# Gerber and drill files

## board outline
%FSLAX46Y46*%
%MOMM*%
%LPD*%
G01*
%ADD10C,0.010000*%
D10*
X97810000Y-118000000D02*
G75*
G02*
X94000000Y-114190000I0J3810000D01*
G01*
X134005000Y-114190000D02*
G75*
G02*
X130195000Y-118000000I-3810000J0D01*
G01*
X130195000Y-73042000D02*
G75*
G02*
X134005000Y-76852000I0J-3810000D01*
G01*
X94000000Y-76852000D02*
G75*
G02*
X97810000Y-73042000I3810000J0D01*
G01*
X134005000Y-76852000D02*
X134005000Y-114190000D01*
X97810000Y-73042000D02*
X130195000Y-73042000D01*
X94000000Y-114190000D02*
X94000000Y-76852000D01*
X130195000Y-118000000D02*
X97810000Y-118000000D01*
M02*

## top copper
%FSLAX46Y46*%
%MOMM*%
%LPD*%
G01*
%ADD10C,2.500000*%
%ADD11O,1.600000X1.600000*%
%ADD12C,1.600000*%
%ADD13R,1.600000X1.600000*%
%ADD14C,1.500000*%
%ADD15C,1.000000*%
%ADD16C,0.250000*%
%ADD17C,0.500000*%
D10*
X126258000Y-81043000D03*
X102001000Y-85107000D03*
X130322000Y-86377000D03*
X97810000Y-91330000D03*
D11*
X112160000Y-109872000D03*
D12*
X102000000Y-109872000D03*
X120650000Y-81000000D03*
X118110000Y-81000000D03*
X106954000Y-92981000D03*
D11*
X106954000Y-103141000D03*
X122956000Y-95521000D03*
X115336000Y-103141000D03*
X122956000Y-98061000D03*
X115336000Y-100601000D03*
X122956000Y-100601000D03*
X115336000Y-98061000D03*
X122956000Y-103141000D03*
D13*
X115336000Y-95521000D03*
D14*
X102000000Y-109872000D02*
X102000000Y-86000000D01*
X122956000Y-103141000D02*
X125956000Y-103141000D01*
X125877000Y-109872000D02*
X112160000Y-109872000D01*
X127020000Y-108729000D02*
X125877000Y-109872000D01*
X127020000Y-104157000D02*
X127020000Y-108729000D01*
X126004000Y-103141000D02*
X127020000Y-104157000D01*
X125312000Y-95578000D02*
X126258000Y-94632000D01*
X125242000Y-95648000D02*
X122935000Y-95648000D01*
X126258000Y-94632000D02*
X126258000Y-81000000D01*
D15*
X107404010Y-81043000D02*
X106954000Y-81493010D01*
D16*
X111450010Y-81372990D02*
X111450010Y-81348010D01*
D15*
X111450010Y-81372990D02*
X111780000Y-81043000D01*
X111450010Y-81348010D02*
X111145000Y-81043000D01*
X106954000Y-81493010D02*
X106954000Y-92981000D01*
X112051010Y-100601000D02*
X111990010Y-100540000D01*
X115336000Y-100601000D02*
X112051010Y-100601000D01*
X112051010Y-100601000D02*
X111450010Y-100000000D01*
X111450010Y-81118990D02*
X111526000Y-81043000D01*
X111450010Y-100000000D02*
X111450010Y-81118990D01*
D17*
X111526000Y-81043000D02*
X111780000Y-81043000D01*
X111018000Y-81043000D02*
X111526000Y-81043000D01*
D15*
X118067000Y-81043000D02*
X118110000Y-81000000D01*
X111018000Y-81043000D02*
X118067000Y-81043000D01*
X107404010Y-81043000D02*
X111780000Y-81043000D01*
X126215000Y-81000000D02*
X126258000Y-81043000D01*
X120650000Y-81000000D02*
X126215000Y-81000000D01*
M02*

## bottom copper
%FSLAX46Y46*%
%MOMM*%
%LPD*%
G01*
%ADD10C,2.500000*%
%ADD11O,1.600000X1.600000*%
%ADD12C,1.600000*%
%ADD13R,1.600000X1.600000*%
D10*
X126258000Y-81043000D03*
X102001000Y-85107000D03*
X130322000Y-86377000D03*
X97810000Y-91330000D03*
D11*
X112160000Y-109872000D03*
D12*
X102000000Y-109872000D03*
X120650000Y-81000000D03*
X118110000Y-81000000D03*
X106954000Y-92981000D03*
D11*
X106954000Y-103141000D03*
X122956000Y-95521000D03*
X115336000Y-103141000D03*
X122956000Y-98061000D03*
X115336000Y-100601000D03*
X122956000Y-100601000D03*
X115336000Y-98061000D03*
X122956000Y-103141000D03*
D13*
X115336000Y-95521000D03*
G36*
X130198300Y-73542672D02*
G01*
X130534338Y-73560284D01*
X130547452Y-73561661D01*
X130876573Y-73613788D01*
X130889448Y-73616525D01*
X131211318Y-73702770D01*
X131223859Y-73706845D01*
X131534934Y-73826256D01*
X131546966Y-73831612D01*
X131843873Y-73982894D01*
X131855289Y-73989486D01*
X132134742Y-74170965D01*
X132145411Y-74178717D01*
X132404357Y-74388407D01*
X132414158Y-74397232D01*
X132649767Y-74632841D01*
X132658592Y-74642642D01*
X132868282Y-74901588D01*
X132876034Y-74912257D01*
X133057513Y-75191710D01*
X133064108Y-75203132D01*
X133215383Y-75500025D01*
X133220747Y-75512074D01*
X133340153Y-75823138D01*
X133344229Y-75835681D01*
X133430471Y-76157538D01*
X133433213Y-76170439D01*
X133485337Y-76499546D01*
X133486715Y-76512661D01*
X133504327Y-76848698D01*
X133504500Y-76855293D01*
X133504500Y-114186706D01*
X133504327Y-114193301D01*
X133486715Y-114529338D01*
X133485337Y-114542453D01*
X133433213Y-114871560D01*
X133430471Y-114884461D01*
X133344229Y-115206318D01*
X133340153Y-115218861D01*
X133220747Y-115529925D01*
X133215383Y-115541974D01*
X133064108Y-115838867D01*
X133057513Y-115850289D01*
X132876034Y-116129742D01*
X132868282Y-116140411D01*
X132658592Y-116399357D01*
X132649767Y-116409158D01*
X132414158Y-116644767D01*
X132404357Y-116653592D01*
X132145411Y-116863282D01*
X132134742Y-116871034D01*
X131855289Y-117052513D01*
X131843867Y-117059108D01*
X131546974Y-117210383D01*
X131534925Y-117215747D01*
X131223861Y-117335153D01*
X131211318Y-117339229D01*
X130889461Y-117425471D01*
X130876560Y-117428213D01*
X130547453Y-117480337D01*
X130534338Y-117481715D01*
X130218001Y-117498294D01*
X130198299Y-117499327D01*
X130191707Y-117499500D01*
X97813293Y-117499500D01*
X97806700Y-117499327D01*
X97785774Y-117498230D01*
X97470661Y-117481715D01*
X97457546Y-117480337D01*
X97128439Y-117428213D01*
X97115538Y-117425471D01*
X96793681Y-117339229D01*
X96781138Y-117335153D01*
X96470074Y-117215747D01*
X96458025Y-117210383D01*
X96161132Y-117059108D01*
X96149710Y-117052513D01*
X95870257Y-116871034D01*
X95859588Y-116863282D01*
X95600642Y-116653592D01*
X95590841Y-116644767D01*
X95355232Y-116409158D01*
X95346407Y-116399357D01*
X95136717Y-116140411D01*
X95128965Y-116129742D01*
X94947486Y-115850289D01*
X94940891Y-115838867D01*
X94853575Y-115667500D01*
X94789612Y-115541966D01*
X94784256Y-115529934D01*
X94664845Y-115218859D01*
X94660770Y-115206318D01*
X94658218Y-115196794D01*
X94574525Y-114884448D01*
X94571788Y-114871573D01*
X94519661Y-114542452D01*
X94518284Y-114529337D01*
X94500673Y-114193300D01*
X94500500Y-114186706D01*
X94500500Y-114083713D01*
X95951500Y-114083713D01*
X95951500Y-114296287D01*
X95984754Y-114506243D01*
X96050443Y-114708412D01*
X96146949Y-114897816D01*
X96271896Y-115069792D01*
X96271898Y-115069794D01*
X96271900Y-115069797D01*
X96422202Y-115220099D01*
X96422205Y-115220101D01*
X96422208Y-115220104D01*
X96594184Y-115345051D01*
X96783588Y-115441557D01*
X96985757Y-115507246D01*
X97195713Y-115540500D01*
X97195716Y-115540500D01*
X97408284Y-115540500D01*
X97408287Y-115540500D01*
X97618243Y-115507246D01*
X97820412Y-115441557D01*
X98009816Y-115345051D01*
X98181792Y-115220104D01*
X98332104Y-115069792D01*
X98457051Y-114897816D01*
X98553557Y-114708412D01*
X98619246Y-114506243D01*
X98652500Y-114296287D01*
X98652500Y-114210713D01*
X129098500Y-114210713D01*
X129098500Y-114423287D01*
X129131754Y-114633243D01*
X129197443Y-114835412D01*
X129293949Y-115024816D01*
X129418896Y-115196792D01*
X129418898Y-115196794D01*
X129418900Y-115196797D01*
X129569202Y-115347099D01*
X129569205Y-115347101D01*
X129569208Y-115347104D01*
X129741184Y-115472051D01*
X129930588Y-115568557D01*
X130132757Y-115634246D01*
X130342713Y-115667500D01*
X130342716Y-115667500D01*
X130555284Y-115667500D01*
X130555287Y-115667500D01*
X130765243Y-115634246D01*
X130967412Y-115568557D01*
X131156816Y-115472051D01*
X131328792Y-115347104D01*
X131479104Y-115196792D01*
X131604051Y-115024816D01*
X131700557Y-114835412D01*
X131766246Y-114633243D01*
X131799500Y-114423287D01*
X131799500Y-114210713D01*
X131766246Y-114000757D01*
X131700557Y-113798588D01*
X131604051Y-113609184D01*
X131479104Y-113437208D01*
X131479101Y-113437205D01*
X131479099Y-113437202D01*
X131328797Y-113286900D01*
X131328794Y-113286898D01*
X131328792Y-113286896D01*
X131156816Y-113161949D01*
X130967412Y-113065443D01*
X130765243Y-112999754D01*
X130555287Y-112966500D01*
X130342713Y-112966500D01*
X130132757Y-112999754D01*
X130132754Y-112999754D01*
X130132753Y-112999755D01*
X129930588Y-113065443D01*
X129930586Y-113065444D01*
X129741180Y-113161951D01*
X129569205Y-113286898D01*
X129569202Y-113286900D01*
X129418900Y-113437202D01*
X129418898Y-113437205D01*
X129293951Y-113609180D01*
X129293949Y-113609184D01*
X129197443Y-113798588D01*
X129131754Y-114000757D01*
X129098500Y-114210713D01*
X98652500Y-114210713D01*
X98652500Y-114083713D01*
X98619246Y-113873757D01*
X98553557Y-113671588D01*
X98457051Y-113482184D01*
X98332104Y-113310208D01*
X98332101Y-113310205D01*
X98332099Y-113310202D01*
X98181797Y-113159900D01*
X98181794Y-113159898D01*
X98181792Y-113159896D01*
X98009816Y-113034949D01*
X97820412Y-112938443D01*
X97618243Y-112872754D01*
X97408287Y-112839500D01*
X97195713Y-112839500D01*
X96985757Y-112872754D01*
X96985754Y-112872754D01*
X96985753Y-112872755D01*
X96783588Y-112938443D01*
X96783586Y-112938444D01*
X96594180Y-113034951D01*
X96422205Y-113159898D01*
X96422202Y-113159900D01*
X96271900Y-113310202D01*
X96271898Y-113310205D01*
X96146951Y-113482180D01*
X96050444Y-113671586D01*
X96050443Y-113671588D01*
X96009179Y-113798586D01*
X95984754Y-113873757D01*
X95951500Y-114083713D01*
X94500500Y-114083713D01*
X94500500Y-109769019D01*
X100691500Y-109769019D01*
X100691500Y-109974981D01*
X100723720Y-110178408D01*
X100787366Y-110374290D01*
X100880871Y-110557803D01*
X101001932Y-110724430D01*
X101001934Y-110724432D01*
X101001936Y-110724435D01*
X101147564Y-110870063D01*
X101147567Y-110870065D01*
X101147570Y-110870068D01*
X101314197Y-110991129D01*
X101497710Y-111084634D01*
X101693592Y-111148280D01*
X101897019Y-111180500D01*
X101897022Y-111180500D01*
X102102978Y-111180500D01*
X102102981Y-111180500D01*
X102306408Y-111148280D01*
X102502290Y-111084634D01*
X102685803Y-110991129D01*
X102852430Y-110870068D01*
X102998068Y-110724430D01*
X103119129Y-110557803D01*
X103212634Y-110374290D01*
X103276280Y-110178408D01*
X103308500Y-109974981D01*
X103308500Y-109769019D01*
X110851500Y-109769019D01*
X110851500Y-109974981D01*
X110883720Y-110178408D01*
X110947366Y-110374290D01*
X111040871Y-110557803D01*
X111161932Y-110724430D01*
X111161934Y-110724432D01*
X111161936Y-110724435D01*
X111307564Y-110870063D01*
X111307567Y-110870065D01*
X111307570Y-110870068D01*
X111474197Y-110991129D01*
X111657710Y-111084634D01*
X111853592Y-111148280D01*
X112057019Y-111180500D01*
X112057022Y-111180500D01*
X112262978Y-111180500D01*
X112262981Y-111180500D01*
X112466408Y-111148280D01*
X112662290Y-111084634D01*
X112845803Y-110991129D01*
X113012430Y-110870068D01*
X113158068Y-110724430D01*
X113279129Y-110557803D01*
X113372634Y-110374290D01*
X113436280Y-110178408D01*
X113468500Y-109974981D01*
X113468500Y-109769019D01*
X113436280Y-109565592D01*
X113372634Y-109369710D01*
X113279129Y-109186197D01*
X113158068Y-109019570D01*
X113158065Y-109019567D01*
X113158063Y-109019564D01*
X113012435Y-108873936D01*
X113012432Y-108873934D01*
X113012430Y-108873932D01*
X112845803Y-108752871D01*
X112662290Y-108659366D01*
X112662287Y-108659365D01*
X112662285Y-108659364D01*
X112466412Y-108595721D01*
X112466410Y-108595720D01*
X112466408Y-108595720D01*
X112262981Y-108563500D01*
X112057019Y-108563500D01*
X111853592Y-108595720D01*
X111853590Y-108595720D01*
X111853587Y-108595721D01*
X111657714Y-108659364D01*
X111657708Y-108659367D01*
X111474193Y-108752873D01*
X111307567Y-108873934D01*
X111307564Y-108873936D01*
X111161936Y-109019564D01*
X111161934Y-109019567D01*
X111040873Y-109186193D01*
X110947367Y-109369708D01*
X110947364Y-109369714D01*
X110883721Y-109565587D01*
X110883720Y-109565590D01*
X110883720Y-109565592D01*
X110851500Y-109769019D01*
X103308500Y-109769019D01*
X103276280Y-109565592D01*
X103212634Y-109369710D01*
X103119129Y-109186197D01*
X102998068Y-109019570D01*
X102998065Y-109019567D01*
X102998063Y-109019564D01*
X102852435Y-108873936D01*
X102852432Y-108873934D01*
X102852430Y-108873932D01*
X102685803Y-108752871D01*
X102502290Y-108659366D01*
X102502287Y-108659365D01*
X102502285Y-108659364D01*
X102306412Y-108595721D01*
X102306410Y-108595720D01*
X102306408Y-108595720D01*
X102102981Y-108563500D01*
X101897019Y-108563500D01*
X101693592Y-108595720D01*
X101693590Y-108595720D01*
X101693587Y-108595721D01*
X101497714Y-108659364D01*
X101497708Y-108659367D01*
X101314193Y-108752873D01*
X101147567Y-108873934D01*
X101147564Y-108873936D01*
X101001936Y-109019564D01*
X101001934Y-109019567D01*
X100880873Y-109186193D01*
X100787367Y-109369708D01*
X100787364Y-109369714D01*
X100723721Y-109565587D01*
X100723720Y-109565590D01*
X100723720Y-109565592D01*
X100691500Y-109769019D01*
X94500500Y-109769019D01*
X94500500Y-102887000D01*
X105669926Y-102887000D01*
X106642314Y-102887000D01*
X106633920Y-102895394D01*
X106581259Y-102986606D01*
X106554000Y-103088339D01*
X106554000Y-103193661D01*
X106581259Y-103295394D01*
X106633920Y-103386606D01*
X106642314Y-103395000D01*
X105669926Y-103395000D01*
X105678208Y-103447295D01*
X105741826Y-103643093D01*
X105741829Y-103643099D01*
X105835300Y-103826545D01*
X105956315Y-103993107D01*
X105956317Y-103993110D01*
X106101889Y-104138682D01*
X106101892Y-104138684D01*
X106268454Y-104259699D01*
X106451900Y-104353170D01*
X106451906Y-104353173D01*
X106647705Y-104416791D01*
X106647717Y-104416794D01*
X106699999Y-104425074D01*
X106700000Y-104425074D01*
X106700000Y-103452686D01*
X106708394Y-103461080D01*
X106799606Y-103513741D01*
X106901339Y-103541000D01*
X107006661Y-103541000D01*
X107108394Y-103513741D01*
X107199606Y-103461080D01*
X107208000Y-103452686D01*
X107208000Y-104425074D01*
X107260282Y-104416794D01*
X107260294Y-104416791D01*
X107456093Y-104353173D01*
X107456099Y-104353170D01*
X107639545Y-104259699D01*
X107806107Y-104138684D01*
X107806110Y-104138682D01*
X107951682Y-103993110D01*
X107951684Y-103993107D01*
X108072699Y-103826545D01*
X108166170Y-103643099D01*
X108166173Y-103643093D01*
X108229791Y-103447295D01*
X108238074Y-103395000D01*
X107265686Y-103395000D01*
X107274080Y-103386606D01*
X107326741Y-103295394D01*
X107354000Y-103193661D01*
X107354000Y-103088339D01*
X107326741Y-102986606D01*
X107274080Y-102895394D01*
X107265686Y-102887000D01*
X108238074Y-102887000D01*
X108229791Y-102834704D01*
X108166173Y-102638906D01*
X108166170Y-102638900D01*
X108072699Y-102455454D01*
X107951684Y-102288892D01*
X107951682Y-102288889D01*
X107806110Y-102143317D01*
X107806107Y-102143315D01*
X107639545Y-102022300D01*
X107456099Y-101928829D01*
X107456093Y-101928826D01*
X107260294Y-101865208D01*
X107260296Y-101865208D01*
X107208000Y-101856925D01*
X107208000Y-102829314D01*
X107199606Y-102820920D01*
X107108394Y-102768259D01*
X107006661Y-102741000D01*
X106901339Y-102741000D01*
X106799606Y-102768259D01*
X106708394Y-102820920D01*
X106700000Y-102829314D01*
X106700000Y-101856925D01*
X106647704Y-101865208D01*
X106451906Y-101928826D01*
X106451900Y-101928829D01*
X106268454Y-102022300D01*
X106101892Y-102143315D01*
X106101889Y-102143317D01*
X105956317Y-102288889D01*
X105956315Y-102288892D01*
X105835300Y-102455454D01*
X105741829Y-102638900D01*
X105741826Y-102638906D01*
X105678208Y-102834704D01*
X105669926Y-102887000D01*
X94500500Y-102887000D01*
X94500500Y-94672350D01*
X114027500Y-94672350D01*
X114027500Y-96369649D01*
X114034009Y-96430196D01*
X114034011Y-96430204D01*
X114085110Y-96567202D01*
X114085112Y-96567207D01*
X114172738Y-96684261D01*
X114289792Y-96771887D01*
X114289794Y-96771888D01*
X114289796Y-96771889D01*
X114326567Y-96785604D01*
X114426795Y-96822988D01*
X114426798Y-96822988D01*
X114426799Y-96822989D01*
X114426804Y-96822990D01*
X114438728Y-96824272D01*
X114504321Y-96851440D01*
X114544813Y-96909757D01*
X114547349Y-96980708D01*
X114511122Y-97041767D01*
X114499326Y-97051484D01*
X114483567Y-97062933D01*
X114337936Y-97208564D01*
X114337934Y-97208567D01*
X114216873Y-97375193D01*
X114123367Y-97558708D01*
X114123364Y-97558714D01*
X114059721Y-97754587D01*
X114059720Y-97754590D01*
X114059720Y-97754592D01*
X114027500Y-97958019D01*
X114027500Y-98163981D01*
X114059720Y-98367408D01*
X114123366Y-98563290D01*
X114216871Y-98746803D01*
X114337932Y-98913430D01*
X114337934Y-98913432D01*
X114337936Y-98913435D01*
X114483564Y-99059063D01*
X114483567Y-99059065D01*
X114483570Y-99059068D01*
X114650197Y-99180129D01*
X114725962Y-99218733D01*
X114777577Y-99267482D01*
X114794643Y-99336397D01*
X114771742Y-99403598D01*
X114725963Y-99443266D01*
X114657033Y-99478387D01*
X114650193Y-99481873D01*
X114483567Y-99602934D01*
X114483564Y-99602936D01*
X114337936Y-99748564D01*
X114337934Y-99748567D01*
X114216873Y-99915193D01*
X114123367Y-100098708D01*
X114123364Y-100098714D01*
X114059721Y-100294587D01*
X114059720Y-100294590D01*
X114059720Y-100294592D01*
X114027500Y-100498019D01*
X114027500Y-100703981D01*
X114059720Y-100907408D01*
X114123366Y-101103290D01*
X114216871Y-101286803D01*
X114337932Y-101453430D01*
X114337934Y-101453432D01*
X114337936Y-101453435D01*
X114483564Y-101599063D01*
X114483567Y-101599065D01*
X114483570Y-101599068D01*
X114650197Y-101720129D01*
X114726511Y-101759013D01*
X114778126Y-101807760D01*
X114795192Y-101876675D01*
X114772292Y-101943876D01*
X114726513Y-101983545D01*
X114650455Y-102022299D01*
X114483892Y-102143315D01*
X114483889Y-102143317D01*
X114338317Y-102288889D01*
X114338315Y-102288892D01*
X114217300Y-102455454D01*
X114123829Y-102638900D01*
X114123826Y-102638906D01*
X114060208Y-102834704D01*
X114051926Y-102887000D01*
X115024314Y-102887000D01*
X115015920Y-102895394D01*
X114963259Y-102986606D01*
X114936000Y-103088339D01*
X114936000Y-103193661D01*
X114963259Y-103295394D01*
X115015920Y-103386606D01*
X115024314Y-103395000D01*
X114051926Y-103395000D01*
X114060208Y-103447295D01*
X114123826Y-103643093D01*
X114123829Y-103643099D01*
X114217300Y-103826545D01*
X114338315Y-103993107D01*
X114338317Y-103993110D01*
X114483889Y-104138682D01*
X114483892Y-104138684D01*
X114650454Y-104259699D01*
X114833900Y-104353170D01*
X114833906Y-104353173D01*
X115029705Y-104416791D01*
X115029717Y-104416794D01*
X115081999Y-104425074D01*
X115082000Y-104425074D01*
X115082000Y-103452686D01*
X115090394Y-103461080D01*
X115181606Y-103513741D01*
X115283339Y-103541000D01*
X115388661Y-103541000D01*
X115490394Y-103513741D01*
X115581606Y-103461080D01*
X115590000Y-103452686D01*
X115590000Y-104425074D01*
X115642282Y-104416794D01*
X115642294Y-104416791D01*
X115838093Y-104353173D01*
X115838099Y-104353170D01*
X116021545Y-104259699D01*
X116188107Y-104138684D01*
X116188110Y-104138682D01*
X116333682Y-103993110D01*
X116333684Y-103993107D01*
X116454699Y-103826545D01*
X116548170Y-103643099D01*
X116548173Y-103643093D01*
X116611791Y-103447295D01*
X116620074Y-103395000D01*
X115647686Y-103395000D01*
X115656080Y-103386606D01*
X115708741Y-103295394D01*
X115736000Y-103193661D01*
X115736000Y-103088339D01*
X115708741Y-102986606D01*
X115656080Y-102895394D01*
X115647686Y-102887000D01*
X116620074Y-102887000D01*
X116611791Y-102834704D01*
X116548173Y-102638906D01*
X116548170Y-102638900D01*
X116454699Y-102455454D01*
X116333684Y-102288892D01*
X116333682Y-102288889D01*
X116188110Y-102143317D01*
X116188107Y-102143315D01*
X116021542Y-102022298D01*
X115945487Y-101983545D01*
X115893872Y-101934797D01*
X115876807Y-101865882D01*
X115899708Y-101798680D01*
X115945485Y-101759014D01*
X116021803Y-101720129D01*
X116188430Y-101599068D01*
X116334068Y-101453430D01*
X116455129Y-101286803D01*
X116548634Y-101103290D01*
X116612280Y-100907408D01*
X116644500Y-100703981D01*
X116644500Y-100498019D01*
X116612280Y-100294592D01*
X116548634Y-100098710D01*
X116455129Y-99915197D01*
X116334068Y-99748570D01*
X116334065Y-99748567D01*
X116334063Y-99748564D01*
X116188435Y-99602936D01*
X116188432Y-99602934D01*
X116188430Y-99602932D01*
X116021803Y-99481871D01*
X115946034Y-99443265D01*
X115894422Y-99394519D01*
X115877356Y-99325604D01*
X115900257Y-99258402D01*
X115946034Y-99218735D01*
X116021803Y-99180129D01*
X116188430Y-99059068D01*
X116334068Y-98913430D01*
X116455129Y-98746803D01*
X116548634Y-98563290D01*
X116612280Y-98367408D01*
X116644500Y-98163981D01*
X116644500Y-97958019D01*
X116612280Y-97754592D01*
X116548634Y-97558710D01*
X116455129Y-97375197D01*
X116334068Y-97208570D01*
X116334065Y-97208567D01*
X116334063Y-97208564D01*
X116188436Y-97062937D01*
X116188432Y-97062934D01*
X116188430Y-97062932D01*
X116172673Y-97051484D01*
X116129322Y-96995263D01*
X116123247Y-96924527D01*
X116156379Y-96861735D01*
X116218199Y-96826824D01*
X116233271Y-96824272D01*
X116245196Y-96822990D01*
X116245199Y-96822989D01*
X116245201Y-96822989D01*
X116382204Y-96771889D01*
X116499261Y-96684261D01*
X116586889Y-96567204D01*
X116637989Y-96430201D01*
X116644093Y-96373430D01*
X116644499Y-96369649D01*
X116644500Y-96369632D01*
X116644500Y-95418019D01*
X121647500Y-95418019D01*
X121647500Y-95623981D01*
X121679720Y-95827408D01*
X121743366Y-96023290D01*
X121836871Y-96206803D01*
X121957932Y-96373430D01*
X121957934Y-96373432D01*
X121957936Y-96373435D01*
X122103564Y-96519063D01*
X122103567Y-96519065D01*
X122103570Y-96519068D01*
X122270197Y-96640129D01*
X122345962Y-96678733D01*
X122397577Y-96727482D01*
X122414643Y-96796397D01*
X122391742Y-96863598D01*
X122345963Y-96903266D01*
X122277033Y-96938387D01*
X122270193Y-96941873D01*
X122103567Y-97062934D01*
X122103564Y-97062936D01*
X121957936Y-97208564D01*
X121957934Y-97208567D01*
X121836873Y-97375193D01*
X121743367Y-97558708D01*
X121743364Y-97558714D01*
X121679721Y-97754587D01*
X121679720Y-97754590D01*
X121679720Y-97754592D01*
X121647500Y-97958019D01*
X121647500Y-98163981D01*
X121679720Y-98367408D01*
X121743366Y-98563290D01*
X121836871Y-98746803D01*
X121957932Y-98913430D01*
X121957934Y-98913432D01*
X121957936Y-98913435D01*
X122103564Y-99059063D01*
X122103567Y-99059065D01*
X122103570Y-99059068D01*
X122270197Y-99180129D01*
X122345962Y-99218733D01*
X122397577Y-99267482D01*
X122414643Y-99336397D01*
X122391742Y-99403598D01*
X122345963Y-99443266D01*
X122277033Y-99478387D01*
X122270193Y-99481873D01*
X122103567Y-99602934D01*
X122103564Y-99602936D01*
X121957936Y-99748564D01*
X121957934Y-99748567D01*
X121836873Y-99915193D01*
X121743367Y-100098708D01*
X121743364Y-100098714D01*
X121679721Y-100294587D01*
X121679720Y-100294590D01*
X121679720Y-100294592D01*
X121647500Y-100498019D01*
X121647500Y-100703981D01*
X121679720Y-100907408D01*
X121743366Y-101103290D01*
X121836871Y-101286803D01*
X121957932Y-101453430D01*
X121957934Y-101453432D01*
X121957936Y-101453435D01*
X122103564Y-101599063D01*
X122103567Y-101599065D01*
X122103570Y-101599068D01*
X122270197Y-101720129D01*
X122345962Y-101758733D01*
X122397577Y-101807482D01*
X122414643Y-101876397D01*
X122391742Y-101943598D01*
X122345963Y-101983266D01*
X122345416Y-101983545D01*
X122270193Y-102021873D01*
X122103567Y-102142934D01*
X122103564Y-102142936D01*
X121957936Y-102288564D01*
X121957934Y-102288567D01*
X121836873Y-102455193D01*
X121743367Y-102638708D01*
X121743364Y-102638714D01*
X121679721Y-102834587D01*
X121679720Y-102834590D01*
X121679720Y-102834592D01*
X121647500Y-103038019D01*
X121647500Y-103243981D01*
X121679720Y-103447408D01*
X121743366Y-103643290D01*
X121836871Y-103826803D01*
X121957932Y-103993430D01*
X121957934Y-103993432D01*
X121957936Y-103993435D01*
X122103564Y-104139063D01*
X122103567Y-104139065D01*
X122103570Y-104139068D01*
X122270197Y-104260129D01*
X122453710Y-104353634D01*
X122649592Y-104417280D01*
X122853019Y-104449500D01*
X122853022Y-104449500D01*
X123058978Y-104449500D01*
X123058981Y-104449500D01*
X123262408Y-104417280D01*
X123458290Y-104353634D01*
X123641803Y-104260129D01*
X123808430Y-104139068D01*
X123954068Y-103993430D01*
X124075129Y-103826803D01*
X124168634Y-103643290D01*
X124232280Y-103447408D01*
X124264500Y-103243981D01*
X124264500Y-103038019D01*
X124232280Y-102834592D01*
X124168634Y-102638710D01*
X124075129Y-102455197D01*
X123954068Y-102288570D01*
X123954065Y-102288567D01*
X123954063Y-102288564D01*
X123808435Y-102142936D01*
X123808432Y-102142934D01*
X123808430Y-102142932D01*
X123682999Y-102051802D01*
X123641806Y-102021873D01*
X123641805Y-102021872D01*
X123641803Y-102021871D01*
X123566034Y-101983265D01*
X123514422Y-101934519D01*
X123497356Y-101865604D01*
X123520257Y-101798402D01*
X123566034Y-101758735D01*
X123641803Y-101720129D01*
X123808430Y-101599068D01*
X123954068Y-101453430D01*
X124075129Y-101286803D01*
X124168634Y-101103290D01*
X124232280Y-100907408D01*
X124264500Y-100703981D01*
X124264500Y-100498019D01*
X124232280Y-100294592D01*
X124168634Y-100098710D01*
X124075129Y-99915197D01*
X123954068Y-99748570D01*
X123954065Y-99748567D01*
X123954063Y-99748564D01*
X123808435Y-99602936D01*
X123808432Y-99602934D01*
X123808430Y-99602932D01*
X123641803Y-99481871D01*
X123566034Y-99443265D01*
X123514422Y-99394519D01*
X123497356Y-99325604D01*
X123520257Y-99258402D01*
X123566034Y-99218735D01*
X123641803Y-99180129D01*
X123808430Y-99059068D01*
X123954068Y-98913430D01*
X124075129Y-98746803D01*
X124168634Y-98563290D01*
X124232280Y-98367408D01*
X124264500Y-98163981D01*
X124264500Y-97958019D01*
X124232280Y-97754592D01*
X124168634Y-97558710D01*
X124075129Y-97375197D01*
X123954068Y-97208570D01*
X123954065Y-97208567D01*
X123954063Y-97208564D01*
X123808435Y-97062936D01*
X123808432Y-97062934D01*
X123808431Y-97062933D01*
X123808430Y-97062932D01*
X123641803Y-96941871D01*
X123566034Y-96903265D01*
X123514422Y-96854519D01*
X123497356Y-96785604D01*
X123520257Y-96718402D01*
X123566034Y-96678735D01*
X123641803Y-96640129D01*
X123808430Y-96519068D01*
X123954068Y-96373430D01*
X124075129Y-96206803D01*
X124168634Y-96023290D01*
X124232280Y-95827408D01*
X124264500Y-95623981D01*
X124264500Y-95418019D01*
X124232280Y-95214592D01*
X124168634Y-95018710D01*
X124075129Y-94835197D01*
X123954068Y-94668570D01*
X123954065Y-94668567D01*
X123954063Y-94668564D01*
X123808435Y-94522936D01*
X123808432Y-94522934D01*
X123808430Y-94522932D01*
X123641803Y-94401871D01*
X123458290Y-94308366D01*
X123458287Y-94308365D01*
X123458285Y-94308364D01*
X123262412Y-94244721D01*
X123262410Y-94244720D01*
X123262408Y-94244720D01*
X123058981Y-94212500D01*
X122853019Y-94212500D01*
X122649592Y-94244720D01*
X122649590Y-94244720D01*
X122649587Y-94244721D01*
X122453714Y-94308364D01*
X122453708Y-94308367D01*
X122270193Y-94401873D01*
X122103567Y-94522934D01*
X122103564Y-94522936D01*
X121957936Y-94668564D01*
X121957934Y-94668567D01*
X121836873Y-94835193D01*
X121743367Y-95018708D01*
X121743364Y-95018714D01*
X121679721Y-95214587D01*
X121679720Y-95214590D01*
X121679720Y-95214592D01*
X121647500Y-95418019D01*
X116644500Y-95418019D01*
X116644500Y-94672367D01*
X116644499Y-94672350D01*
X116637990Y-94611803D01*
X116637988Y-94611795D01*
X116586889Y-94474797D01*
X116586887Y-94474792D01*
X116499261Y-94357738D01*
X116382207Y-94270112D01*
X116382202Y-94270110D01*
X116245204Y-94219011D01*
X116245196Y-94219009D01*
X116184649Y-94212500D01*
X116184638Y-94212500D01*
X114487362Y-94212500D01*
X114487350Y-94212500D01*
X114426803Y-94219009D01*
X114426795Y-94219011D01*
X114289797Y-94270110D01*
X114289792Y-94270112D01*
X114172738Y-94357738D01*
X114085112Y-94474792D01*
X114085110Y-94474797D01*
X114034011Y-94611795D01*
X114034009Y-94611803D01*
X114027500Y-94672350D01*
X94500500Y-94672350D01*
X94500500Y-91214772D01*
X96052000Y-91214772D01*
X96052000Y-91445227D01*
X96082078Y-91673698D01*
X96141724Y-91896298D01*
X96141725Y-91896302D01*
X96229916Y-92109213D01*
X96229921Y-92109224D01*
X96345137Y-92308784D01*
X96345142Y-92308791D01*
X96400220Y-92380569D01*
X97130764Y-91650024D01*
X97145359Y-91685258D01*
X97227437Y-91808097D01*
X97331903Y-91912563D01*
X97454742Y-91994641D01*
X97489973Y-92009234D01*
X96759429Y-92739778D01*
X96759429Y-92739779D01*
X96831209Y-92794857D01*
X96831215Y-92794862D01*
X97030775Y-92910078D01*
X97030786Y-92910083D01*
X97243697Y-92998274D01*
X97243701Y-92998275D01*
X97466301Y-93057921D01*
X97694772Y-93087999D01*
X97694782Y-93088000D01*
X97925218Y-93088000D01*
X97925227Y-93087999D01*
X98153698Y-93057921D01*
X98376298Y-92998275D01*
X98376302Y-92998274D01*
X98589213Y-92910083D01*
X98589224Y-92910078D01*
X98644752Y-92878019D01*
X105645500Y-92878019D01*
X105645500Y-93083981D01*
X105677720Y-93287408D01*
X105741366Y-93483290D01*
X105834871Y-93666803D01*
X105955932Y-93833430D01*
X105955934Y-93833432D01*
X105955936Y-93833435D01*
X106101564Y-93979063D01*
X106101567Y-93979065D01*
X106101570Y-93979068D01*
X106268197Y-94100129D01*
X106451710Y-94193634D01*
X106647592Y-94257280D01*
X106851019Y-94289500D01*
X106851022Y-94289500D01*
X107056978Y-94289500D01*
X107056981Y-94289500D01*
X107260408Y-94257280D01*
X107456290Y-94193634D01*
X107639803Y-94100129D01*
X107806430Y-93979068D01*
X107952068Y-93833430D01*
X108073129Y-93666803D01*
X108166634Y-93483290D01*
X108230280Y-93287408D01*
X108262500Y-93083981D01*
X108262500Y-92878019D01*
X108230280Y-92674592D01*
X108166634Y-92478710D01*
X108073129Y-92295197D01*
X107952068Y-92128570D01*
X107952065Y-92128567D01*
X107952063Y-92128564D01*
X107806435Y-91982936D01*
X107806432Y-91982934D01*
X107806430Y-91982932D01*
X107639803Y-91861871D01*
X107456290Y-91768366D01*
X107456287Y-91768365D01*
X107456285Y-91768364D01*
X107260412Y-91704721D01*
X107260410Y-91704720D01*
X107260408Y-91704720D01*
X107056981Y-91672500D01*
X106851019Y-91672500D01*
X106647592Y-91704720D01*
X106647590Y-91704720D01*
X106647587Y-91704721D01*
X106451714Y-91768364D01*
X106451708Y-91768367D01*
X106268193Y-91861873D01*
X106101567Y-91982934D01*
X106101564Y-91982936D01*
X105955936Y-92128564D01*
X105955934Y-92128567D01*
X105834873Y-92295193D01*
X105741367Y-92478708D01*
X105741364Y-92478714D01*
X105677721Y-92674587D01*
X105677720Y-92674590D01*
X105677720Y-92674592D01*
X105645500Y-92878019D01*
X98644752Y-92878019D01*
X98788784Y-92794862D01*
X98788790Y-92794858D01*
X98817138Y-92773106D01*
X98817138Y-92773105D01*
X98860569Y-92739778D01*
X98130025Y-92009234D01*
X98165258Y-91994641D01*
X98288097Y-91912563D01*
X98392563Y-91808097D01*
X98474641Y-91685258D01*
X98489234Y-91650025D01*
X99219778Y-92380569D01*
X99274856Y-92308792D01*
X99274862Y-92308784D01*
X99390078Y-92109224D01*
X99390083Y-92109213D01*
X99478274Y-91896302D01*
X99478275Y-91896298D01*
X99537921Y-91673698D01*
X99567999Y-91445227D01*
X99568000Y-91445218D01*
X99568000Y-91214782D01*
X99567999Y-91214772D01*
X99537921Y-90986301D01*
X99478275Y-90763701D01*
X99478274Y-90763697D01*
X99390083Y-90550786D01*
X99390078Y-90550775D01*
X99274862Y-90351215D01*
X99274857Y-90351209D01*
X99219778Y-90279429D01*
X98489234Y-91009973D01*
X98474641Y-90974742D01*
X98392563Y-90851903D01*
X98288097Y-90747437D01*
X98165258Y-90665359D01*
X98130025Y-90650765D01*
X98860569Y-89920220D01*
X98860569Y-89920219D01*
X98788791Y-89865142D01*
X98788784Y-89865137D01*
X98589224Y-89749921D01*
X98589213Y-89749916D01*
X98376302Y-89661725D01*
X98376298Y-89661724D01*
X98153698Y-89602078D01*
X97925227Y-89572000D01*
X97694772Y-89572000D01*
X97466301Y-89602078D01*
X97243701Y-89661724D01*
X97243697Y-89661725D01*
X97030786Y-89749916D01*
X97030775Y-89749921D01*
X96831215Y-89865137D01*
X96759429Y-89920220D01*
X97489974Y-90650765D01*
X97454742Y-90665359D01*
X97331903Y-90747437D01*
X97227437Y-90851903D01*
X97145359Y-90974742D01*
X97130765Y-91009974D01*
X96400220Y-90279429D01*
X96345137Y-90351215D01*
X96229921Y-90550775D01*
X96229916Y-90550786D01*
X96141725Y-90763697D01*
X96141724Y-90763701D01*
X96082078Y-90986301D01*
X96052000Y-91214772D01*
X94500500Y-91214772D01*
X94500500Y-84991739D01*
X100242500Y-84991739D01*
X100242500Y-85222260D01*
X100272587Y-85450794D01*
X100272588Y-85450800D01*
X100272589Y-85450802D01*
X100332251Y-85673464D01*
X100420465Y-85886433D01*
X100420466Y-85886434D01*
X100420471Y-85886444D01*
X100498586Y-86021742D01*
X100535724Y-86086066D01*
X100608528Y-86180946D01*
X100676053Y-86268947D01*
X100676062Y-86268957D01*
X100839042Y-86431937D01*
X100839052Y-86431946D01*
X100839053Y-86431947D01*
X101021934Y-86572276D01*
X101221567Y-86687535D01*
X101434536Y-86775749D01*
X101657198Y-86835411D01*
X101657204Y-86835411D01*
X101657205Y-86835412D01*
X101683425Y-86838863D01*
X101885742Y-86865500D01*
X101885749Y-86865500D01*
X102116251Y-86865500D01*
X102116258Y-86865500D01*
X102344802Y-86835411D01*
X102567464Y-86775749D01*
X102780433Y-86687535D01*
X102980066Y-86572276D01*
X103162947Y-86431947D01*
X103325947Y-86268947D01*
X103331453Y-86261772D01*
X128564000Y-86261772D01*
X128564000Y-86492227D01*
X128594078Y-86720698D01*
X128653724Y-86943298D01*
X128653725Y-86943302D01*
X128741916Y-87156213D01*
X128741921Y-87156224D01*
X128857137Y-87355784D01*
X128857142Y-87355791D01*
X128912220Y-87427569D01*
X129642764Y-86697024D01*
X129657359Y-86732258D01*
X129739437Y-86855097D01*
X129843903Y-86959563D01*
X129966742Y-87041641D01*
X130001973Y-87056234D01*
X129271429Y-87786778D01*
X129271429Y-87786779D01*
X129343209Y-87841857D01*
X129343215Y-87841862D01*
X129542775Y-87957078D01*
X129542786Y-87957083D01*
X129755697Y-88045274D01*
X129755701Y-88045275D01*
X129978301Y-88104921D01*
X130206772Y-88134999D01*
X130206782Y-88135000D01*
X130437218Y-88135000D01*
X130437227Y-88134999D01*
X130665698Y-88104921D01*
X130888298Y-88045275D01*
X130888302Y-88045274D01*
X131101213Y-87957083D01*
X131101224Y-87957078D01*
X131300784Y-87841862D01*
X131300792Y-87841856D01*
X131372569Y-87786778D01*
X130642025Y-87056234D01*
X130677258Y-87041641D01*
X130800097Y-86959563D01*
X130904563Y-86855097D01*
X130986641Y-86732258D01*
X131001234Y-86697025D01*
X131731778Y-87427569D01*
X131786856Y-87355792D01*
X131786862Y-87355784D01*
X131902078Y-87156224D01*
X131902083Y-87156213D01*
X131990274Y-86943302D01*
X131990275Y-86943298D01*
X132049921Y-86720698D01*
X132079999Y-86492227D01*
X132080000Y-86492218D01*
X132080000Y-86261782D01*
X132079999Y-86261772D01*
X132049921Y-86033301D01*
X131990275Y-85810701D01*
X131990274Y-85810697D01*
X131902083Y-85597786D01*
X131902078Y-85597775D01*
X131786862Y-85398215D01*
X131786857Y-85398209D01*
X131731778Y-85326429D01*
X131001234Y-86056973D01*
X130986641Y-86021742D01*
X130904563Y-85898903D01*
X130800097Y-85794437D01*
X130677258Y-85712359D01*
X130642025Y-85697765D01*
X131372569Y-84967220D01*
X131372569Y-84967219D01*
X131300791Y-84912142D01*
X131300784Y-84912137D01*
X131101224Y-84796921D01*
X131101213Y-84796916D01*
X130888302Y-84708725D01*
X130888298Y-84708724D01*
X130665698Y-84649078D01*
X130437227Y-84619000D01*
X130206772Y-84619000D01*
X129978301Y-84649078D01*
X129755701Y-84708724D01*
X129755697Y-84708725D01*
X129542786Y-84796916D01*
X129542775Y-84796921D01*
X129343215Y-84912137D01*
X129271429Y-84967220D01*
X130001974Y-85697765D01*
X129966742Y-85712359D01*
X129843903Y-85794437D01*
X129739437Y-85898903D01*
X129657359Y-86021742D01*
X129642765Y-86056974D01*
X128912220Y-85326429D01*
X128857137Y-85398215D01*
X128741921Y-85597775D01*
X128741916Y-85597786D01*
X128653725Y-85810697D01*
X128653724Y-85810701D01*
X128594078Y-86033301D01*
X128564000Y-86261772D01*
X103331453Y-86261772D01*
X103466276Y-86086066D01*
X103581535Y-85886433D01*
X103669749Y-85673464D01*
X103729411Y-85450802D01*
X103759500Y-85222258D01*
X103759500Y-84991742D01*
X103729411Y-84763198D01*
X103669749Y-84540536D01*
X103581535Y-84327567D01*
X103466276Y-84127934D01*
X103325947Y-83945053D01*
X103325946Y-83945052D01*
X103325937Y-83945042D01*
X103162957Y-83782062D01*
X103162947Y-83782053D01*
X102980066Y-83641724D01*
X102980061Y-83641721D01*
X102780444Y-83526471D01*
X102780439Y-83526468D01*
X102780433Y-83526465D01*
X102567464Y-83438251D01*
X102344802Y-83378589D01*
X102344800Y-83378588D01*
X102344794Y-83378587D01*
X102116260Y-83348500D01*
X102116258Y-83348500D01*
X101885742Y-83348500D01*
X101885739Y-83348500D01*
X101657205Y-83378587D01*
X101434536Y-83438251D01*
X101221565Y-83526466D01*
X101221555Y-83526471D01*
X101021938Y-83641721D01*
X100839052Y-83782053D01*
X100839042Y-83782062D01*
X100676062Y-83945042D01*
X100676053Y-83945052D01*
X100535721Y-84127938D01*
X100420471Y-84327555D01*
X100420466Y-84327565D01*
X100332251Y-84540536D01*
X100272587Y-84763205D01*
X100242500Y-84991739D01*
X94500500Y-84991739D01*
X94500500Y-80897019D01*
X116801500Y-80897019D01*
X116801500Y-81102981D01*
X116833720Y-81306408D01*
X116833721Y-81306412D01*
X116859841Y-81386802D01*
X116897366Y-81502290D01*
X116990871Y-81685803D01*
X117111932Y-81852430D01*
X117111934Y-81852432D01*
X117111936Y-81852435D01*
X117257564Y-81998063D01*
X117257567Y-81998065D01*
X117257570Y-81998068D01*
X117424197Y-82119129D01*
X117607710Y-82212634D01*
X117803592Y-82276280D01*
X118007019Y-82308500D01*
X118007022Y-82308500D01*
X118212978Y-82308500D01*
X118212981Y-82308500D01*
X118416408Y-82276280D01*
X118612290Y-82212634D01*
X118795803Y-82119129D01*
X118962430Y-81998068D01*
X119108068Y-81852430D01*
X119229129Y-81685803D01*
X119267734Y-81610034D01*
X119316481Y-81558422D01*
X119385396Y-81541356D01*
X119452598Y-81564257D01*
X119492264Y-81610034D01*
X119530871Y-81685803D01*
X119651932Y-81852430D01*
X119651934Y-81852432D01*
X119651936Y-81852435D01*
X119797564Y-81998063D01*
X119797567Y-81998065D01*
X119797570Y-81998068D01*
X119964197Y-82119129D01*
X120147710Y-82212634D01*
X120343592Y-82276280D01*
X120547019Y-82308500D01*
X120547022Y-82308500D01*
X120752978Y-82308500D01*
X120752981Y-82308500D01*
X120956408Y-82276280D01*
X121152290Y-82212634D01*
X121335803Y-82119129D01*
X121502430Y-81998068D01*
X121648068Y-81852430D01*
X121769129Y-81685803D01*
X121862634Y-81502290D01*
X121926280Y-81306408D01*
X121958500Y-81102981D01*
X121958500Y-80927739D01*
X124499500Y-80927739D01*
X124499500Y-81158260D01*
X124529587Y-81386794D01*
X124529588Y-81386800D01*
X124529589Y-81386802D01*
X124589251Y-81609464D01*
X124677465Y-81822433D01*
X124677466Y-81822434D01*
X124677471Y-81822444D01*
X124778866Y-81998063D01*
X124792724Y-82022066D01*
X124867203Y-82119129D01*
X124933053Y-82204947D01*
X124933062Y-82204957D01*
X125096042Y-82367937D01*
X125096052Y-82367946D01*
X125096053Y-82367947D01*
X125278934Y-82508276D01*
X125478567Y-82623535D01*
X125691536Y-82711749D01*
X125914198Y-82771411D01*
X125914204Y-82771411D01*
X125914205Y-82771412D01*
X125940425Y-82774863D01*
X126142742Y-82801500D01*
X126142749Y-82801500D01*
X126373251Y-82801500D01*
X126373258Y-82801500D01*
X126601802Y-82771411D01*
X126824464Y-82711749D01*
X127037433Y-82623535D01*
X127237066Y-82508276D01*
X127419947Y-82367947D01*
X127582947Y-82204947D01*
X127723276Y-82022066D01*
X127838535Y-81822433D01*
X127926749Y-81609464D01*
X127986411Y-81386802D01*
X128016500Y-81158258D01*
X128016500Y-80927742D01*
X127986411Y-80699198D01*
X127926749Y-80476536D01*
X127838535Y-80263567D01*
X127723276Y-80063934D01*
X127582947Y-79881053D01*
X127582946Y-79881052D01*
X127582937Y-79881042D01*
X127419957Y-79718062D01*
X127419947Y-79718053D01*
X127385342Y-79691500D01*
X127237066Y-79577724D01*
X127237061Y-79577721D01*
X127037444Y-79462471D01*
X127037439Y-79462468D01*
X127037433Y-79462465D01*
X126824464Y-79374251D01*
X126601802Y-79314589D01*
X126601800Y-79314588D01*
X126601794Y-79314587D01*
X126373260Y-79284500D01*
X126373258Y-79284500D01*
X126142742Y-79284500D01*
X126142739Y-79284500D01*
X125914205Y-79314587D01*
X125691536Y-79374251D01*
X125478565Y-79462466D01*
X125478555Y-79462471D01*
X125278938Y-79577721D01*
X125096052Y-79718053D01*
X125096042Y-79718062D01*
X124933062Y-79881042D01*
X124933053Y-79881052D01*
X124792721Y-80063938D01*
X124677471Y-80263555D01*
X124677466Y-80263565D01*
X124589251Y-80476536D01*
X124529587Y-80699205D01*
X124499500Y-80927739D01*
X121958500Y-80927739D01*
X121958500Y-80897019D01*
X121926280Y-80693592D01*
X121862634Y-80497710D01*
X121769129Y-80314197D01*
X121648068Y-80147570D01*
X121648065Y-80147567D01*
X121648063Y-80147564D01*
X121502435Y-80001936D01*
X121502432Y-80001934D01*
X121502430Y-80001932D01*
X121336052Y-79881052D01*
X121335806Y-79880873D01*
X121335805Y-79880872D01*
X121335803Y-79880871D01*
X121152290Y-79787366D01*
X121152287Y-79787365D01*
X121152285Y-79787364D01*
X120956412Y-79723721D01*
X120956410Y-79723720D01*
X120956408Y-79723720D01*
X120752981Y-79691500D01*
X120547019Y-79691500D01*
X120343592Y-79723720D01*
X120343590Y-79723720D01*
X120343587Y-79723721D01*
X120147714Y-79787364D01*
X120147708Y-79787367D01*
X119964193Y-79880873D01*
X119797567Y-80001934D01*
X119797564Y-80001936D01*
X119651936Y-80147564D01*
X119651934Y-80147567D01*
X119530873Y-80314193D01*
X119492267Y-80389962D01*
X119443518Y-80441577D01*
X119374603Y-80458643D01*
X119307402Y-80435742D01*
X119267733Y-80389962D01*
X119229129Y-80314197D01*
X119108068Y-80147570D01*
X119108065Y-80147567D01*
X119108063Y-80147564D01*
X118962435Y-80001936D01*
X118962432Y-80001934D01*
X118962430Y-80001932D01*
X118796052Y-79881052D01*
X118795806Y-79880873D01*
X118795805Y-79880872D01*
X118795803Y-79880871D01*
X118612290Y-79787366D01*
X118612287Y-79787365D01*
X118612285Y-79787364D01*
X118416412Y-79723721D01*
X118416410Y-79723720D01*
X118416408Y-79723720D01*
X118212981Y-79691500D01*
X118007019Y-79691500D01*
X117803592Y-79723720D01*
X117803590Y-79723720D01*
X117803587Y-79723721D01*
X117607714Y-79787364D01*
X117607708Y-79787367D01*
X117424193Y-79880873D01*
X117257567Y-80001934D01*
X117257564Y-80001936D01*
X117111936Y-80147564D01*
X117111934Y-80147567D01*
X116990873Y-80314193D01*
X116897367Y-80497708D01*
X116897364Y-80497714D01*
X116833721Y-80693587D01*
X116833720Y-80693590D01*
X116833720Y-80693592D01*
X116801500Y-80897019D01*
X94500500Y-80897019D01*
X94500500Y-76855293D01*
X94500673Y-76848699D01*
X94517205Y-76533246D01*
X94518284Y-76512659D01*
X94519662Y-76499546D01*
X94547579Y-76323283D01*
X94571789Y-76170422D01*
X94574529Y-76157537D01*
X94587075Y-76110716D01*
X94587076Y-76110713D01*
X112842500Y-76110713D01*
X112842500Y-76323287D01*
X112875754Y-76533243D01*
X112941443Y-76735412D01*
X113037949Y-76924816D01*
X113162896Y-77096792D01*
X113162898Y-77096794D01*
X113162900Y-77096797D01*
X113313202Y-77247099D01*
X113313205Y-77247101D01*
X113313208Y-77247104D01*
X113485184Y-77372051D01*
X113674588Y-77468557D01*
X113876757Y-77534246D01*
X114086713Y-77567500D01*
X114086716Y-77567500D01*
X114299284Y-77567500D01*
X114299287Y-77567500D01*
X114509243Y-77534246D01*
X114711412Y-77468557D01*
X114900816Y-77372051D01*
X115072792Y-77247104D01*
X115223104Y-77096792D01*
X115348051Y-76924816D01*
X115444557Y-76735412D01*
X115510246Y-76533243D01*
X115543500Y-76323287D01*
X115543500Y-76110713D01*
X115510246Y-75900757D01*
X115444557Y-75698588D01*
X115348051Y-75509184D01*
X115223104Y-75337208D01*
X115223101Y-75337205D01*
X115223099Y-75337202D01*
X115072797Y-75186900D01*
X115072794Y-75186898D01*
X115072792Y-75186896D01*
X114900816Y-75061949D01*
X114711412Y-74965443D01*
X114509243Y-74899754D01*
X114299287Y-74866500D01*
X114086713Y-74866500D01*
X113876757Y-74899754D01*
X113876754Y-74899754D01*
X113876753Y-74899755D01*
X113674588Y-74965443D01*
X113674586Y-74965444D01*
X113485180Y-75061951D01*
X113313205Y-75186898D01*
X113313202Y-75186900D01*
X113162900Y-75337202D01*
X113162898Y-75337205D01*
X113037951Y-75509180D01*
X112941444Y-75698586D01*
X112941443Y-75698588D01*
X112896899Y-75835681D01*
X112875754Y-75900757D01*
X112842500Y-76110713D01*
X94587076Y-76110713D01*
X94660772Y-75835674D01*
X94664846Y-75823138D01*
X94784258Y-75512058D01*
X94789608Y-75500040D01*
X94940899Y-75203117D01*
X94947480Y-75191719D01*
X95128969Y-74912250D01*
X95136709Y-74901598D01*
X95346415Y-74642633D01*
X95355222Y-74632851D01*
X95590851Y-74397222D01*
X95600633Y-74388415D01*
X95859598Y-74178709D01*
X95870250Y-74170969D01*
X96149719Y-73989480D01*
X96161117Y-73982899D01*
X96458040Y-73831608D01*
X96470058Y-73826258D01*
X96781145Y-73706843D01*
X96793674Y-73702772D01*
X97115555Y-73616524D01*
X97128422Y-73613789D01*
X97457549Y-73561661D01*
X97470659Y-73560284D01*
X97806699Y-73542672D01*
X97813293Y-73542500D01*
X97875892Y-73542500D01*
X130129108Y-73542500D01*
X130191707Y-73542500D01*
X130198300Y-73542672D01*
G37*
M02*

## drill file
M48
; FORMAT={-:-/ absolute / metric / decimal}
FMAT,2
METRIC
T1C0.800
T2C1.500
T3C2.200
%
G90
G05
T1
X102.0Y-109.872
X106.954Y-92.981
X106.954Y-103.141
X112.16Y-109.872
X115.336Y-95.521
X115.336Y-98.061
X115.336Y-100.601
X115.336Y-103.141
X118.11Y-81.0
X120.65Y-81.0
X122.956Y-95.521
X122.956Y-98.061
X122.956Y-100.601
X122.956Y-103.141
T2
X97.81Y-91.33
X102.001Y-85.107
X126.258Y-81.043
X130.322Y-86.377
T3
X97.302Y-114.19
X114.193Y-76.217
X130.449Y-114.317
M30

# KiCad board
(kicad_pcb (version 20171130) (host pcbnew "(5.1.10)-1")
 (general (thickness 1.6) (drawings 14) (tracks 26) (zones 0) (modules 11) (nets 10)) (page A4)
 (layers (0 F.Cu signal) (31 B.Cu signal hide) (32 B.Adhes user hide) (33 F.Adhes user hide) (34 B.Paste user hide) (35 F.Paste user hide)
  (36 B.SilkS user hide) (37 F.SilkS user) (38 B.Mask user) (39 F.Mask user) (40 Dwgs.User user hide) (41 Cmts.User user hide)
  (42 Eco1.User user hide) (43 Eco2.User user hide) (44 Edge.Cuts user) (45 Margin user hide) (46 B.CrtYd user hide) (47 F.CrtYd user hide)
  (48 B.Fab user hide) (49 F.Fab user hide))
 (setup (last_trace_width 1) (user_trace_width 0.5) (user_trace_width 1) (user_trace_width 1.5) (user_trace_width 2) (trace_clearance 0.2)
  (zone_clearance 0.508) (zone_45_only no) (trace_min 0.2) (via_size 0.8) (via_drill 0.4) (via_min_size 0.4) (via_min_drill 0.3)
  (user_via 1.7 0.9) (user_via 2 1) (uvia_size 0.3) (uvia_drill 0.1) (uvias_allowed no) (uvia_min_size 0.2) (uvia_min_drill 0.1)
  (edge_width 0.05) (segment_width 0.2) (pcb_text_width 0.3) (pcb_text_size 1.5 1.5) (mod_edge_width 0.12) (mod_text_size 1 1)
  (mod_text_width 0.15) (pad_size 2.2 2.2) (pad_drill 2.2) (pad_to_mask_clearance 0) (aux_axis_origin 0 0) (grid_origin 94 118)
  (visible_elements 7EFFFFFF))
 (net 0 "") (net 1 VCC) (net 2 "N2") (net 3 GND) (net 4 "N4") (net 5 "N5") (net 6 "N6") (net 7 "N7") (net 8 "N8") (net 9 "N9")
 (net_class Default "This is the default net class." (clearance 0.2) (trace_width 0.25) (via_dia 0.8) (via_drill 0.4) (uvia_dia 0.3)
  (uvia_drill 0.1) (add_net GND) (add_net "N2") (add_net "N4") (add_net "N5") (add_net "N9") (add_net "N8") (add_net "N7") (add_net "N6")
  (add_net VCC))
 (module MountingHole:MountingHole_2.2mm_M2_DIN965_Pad (layer F.Cu) (at 126.258 81.043)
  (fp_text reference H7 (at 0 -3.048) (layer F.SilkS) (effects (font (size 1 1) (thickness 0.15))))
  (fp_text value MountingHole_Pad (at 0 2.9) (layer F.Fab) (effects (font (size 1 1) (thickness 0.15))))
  (pad 1 thru_hole circle (at 0 0) (size 2.5 2.5) (drill 1.5) (layers *.Cu *.Mask) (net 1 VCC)))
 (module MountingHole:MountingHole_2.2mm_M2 (layer F.Cu) (at 97.302 114.19)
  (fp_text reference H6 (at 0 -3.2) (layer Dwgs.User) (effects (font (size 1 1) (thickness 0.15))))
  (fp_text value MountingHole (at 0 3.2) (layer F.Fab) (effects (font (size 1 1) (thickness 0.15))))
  (pad "" np_thru_hole circle (at 0 0) (size 2.2 2.2) (drill 2.2) (layers *.Cu *.Mask)))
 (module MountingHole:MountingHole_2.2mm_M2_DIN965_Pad (layer F.Cu) (at 102.001 85.107)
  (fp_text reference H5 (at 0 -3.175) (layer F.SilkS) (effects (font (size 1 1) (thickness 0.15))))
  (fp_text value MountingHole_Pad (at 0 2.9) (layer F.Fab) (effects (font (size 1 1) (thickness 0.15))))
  (pad 1 thru_hole circle (at 0 0) (size 2.5 2.5) (drill 1.5) (layers *.Cu *.Mask) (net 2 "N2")))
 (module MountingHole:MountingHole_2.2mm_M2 (layer F.Cu) (at 130.449 114.317)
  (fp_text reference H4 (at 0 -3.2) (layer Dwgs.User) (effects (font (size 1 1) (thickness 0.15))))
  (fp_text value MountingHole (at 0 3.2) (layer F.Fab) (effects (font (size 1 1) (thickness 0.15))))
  (pad "" np_thru_hole circle (at 0 0) (size 2.2 2.2) (drill 2.2) (layers *.Cu *.Mask)))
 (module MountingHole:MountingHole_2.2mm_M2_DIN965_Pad (layer F.Cu) (at 130.322 86.377)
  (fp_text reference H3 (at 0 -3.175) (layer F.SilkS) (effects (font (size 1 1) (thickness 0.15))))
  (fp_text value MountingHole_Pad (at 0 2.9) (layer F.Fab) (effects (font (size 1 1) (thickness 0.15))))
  (pad 1 thru_hole circle (at 0 0) (size 2.5 2.5) (drill 1.5) (layers *.Cu *.Mask) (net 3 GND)))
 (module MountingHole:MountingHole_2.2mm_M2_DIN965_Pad (layer F.Cu) (at 97.81 91.33)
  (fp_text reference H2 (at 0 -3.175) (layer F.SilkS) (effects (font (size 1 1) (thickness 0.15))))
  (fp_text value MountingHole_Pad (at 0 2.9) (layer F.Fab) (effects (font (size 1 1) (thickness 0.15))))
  (pad 1 thru_hole circle (at 0 0) (size 2.5 2.5) (drill 1.5) (layers *.Cu *.Mask) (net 3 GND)))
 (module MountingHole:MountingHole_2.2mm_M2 (layer F.Cu) (at 114.193 76.217)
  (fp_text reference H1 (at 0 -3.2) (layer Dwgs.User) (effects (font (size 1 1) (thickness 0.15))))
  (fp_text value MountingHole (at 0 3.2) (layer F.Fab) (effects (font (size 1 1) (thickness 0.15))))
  (pad "" np_thru_hole circle (at 0 0) (size 2.2 2.2) (drill 2.2) (layers *.Cu *.Mask)))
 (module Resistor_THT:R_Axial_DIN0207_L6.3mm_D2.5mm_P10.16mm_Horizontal (layer F.Cu) (at 102 109.872)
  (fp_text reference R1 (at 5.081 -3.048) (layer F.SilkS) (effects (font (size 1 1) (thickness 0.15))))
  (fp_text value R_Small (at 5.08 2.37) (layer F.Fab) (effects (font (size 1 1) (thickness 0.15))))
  (pad 2 thru_hole oval (at 10.16 0) (size 1.6 1.6) (drill 0.8) (layers *.Cu *.Mask) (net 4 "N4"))
  (pad 1 thru_hole circle (at 0 0) (size 1.6 1.6) (drill 0.8) (layers *.Cu *.Mask) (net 2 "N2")))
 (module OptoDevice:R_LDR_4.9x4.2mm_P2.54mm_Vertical (layer F.Cu) (at 118.11 81)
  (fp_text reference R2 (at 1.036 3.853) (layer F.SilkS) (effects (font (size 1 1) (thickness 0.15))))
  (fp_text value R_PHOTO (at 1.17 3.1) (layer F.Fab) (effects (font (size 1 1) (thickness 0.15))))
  (pad 2 thru_hole circle (at 2.54 0) (size 1.6 1.6) (drill 0.8) (layers *.Cu *.Mask) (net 1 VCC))
  (pad 1 thru_hole circle (at 0 0) (size 1.6 1.6) (drill 0.8) (layers *.Cu *.Mask) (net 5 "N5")))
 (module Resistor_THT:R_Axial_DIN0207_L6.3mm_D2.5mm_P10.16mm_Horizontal (layer F.Cu) (at 106.954 92.981 270)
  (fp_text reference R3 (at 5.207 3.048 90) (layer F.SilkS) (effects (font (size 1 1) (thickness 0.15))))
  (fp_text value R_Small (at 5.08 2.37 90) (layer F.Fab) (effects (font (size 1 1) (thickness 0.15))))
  (pad 1 thru_hole circle (at 0 0 270) (size 1.6 1.6) (drill 0.8) (layers *.Cu *.Mask) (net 5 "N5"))
  (pad 2 thru_hole oval (at 10.16 0 270) (size 1.6 1.6) (drill 0.8) (layers *.Cu *.Mask) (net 3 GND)))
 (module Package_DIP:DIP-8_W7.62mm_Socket (layer F.Cu) (at 115.336 95.521)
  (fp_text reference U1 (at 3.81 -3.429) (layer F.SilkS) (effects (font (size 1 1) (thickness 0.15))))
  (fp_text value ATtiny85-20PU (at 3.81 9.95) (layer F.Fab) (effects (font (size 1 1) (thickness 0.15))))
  (pad 8 thru_hole oval (at 7.62 0) (size 1.6 1.6) (drill 0.8) (layers *.Cu *.Mask) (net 1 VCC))
  (pad 4 thru_hole oval (at 0 7.62) (size 1.6 1.6) (drill 0.8) (layers *.Cu *.Mask) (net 3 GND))
  (pad 7 thru_hole oval (at 7.62 2.54) (size 1.6 1.6) (drill 0.8) (layers *.Cu *.Mask) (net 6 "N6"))
  (pad 3 thru_hole oval (at 0 5.08) (size 1.6 1.6) (drill 0.8) (layers *.Cu *.Mask) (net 5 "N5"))
  (pad 6 thru_hole oval (at 7.62 5.08) (size 1.6 1.6) (drill 0.8) (layers *.Cu *.Mask) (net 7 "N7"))
  (pad 2 thru_hole oval (at 0 2.54) (size 1.6 1.6) (drill 0.8) (layers *.Cu *.Mask) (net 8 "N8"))
  (pad 5 thru_hole oval (at 7.62 7.62) (size 1.6 1.6) (drill 0.8) (layers *.Cu *.Mask) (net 4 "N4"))
  (pad 1 thru_hole rect (at 0 0) (size 1.6 1.6) (drill 0.8) (layers *.Cu *.Mask) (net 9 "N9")))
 (gr_arc (start 97.81 114.19) (end 94 114.19) (angle -90) (layer Edge.Cuts) (width 0.01))
 (gr_arc (start 130.195 114.19) (end 130.195 118) (angle -90) (layer Edge.Cuts) (width 0.01))
 (gr_arc (start 130.195 76.852) (end 134.005 76.852) (angle -90) (layer Edge.Cuts) (width 0.01))
 (gr_arc (start 97.81 76.852) (end 97.81 73.042) (angle -90) (layer Edge.Cuts) (width 0.01))
 (gr_line (start 134.005 76.852) (end 134.005 114.19) (layer Edge.Cuts) (width 0.01))
 (gr_line (start 97.81 73.042) (end 130.195 73.042) (layer Edge.Cuts) (width 0.01))
 (gr_line (start 94 114.19) (end 94 76.852) (layer Edge.Cuts) (width 0.01))
 (gr_line (start 130.195 118) (end 97.81 118) (layer Edge.Cuts) (width 0.01))
 (segment (start 102 109.872) (end 102 86) (width 1.5) (layer F.Cu) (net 2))
 (segment (start 122.956 103.141) (end 125.956 103.141) (width 1.5) (layer F.Cu) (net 4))
 (segment (start 125.877 109.872) (end 112.16 109.872) (width 1.5) (layer F.Cu) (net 4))
 (segment (start 127.02 108.729) (end 125.877 109.872) (width 1.5) (layer F.Cu) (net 4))
 (segment (start 127.02 104.157) (end 127.02 108.729) (width 1.5) (layer F.Cu) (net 4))
 (segment (start 126.004 103.141) (end 127.02 104.157) (width 1.5) (layer F.Cu) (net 4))
 (segment (start 125.312 95.578) (end 126.258 94.632) (width 1.5) (layer F.Cu) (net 1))
 (segment (start 125.242 95.648) (end 122.935 95.648) (width 1.5) (layer F.Cu) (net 1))
 (segment (start 126.258 94.632) (end 126.258 81) (width 1.5) (layer F.Cu) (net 1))
 (segment (start 107.40401 81.043) (end 106.954 81.49301) (width 1) (layer F.Cu) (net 5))
 (segment (start 111.45001 81.37299) (end 111.45001 81.34801) (width 0.25) (layer F.Cu) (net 5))
 (segment (start 111.45001 81.37299) (end 111.78 81.043) (width 1) (layer F.Cu) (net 5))
 (segment (start 111.45001 81.34801) (end 111.145 81.043) (width 1) (layer F.Cu) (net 5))
 (segment (start 106.954 81.49301) (end 106.954 92.981) (width 1) (layer F.Cu) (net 5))
 (segment (start 112.05101 100.601) (end 111.99001 100.54) (width 1) (layer F.Cu) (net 5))
 (segment (start 115.336 100.601) (end 112.05101 100.601) (width 1) (layer F.Cu) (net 5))
 (segment (start 112.05101 100.601) (end 111.45001 100) (width 1) (layer F.Cu) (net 5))
 (segment (start 111.45001 81.11899) (end 111.526 81.043) (width 1) (layer F.Cu) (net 5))
 (segment (start 111.45001 100) (end 111.45001 81.11899) (width 1) (layer F.Cu) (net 5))
 (segment (start 111.526 81.043) (end 111.78 81.043) (width 0.5) (layer F.Cu) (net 5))
 (segment (start 111.018 81.043) (end 111.526 81.043) (width 0.5) (layer F.Cu) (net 5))
 (segment (start 118.067 81.043) (end 118.11 81) (width 1) (layer F.Cu) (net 5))
 (segment (start 111.018 81.043) (end 118.067 81.043) (width 1) (layer F.Cu) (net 5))
 (segment (start 107.40401 81.043) (end 111.78 81.043) (width 1) (layer F.Cu) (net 5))
 (segment (start 126.215 81) (end 126.258 81.043) (width 1) (layer F.Cu) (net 1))
 (segment (start 120.65 81) (end 126.215 81) (width 1) (layer F.Cu) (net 1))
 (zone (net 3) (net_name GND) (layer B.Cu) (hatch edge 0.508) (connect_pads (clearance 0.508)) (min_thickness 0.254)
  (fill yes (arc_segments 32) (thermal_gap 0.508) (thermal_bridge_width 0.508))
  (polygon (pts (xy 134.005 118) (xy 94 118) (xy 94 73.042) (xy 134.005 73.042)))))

